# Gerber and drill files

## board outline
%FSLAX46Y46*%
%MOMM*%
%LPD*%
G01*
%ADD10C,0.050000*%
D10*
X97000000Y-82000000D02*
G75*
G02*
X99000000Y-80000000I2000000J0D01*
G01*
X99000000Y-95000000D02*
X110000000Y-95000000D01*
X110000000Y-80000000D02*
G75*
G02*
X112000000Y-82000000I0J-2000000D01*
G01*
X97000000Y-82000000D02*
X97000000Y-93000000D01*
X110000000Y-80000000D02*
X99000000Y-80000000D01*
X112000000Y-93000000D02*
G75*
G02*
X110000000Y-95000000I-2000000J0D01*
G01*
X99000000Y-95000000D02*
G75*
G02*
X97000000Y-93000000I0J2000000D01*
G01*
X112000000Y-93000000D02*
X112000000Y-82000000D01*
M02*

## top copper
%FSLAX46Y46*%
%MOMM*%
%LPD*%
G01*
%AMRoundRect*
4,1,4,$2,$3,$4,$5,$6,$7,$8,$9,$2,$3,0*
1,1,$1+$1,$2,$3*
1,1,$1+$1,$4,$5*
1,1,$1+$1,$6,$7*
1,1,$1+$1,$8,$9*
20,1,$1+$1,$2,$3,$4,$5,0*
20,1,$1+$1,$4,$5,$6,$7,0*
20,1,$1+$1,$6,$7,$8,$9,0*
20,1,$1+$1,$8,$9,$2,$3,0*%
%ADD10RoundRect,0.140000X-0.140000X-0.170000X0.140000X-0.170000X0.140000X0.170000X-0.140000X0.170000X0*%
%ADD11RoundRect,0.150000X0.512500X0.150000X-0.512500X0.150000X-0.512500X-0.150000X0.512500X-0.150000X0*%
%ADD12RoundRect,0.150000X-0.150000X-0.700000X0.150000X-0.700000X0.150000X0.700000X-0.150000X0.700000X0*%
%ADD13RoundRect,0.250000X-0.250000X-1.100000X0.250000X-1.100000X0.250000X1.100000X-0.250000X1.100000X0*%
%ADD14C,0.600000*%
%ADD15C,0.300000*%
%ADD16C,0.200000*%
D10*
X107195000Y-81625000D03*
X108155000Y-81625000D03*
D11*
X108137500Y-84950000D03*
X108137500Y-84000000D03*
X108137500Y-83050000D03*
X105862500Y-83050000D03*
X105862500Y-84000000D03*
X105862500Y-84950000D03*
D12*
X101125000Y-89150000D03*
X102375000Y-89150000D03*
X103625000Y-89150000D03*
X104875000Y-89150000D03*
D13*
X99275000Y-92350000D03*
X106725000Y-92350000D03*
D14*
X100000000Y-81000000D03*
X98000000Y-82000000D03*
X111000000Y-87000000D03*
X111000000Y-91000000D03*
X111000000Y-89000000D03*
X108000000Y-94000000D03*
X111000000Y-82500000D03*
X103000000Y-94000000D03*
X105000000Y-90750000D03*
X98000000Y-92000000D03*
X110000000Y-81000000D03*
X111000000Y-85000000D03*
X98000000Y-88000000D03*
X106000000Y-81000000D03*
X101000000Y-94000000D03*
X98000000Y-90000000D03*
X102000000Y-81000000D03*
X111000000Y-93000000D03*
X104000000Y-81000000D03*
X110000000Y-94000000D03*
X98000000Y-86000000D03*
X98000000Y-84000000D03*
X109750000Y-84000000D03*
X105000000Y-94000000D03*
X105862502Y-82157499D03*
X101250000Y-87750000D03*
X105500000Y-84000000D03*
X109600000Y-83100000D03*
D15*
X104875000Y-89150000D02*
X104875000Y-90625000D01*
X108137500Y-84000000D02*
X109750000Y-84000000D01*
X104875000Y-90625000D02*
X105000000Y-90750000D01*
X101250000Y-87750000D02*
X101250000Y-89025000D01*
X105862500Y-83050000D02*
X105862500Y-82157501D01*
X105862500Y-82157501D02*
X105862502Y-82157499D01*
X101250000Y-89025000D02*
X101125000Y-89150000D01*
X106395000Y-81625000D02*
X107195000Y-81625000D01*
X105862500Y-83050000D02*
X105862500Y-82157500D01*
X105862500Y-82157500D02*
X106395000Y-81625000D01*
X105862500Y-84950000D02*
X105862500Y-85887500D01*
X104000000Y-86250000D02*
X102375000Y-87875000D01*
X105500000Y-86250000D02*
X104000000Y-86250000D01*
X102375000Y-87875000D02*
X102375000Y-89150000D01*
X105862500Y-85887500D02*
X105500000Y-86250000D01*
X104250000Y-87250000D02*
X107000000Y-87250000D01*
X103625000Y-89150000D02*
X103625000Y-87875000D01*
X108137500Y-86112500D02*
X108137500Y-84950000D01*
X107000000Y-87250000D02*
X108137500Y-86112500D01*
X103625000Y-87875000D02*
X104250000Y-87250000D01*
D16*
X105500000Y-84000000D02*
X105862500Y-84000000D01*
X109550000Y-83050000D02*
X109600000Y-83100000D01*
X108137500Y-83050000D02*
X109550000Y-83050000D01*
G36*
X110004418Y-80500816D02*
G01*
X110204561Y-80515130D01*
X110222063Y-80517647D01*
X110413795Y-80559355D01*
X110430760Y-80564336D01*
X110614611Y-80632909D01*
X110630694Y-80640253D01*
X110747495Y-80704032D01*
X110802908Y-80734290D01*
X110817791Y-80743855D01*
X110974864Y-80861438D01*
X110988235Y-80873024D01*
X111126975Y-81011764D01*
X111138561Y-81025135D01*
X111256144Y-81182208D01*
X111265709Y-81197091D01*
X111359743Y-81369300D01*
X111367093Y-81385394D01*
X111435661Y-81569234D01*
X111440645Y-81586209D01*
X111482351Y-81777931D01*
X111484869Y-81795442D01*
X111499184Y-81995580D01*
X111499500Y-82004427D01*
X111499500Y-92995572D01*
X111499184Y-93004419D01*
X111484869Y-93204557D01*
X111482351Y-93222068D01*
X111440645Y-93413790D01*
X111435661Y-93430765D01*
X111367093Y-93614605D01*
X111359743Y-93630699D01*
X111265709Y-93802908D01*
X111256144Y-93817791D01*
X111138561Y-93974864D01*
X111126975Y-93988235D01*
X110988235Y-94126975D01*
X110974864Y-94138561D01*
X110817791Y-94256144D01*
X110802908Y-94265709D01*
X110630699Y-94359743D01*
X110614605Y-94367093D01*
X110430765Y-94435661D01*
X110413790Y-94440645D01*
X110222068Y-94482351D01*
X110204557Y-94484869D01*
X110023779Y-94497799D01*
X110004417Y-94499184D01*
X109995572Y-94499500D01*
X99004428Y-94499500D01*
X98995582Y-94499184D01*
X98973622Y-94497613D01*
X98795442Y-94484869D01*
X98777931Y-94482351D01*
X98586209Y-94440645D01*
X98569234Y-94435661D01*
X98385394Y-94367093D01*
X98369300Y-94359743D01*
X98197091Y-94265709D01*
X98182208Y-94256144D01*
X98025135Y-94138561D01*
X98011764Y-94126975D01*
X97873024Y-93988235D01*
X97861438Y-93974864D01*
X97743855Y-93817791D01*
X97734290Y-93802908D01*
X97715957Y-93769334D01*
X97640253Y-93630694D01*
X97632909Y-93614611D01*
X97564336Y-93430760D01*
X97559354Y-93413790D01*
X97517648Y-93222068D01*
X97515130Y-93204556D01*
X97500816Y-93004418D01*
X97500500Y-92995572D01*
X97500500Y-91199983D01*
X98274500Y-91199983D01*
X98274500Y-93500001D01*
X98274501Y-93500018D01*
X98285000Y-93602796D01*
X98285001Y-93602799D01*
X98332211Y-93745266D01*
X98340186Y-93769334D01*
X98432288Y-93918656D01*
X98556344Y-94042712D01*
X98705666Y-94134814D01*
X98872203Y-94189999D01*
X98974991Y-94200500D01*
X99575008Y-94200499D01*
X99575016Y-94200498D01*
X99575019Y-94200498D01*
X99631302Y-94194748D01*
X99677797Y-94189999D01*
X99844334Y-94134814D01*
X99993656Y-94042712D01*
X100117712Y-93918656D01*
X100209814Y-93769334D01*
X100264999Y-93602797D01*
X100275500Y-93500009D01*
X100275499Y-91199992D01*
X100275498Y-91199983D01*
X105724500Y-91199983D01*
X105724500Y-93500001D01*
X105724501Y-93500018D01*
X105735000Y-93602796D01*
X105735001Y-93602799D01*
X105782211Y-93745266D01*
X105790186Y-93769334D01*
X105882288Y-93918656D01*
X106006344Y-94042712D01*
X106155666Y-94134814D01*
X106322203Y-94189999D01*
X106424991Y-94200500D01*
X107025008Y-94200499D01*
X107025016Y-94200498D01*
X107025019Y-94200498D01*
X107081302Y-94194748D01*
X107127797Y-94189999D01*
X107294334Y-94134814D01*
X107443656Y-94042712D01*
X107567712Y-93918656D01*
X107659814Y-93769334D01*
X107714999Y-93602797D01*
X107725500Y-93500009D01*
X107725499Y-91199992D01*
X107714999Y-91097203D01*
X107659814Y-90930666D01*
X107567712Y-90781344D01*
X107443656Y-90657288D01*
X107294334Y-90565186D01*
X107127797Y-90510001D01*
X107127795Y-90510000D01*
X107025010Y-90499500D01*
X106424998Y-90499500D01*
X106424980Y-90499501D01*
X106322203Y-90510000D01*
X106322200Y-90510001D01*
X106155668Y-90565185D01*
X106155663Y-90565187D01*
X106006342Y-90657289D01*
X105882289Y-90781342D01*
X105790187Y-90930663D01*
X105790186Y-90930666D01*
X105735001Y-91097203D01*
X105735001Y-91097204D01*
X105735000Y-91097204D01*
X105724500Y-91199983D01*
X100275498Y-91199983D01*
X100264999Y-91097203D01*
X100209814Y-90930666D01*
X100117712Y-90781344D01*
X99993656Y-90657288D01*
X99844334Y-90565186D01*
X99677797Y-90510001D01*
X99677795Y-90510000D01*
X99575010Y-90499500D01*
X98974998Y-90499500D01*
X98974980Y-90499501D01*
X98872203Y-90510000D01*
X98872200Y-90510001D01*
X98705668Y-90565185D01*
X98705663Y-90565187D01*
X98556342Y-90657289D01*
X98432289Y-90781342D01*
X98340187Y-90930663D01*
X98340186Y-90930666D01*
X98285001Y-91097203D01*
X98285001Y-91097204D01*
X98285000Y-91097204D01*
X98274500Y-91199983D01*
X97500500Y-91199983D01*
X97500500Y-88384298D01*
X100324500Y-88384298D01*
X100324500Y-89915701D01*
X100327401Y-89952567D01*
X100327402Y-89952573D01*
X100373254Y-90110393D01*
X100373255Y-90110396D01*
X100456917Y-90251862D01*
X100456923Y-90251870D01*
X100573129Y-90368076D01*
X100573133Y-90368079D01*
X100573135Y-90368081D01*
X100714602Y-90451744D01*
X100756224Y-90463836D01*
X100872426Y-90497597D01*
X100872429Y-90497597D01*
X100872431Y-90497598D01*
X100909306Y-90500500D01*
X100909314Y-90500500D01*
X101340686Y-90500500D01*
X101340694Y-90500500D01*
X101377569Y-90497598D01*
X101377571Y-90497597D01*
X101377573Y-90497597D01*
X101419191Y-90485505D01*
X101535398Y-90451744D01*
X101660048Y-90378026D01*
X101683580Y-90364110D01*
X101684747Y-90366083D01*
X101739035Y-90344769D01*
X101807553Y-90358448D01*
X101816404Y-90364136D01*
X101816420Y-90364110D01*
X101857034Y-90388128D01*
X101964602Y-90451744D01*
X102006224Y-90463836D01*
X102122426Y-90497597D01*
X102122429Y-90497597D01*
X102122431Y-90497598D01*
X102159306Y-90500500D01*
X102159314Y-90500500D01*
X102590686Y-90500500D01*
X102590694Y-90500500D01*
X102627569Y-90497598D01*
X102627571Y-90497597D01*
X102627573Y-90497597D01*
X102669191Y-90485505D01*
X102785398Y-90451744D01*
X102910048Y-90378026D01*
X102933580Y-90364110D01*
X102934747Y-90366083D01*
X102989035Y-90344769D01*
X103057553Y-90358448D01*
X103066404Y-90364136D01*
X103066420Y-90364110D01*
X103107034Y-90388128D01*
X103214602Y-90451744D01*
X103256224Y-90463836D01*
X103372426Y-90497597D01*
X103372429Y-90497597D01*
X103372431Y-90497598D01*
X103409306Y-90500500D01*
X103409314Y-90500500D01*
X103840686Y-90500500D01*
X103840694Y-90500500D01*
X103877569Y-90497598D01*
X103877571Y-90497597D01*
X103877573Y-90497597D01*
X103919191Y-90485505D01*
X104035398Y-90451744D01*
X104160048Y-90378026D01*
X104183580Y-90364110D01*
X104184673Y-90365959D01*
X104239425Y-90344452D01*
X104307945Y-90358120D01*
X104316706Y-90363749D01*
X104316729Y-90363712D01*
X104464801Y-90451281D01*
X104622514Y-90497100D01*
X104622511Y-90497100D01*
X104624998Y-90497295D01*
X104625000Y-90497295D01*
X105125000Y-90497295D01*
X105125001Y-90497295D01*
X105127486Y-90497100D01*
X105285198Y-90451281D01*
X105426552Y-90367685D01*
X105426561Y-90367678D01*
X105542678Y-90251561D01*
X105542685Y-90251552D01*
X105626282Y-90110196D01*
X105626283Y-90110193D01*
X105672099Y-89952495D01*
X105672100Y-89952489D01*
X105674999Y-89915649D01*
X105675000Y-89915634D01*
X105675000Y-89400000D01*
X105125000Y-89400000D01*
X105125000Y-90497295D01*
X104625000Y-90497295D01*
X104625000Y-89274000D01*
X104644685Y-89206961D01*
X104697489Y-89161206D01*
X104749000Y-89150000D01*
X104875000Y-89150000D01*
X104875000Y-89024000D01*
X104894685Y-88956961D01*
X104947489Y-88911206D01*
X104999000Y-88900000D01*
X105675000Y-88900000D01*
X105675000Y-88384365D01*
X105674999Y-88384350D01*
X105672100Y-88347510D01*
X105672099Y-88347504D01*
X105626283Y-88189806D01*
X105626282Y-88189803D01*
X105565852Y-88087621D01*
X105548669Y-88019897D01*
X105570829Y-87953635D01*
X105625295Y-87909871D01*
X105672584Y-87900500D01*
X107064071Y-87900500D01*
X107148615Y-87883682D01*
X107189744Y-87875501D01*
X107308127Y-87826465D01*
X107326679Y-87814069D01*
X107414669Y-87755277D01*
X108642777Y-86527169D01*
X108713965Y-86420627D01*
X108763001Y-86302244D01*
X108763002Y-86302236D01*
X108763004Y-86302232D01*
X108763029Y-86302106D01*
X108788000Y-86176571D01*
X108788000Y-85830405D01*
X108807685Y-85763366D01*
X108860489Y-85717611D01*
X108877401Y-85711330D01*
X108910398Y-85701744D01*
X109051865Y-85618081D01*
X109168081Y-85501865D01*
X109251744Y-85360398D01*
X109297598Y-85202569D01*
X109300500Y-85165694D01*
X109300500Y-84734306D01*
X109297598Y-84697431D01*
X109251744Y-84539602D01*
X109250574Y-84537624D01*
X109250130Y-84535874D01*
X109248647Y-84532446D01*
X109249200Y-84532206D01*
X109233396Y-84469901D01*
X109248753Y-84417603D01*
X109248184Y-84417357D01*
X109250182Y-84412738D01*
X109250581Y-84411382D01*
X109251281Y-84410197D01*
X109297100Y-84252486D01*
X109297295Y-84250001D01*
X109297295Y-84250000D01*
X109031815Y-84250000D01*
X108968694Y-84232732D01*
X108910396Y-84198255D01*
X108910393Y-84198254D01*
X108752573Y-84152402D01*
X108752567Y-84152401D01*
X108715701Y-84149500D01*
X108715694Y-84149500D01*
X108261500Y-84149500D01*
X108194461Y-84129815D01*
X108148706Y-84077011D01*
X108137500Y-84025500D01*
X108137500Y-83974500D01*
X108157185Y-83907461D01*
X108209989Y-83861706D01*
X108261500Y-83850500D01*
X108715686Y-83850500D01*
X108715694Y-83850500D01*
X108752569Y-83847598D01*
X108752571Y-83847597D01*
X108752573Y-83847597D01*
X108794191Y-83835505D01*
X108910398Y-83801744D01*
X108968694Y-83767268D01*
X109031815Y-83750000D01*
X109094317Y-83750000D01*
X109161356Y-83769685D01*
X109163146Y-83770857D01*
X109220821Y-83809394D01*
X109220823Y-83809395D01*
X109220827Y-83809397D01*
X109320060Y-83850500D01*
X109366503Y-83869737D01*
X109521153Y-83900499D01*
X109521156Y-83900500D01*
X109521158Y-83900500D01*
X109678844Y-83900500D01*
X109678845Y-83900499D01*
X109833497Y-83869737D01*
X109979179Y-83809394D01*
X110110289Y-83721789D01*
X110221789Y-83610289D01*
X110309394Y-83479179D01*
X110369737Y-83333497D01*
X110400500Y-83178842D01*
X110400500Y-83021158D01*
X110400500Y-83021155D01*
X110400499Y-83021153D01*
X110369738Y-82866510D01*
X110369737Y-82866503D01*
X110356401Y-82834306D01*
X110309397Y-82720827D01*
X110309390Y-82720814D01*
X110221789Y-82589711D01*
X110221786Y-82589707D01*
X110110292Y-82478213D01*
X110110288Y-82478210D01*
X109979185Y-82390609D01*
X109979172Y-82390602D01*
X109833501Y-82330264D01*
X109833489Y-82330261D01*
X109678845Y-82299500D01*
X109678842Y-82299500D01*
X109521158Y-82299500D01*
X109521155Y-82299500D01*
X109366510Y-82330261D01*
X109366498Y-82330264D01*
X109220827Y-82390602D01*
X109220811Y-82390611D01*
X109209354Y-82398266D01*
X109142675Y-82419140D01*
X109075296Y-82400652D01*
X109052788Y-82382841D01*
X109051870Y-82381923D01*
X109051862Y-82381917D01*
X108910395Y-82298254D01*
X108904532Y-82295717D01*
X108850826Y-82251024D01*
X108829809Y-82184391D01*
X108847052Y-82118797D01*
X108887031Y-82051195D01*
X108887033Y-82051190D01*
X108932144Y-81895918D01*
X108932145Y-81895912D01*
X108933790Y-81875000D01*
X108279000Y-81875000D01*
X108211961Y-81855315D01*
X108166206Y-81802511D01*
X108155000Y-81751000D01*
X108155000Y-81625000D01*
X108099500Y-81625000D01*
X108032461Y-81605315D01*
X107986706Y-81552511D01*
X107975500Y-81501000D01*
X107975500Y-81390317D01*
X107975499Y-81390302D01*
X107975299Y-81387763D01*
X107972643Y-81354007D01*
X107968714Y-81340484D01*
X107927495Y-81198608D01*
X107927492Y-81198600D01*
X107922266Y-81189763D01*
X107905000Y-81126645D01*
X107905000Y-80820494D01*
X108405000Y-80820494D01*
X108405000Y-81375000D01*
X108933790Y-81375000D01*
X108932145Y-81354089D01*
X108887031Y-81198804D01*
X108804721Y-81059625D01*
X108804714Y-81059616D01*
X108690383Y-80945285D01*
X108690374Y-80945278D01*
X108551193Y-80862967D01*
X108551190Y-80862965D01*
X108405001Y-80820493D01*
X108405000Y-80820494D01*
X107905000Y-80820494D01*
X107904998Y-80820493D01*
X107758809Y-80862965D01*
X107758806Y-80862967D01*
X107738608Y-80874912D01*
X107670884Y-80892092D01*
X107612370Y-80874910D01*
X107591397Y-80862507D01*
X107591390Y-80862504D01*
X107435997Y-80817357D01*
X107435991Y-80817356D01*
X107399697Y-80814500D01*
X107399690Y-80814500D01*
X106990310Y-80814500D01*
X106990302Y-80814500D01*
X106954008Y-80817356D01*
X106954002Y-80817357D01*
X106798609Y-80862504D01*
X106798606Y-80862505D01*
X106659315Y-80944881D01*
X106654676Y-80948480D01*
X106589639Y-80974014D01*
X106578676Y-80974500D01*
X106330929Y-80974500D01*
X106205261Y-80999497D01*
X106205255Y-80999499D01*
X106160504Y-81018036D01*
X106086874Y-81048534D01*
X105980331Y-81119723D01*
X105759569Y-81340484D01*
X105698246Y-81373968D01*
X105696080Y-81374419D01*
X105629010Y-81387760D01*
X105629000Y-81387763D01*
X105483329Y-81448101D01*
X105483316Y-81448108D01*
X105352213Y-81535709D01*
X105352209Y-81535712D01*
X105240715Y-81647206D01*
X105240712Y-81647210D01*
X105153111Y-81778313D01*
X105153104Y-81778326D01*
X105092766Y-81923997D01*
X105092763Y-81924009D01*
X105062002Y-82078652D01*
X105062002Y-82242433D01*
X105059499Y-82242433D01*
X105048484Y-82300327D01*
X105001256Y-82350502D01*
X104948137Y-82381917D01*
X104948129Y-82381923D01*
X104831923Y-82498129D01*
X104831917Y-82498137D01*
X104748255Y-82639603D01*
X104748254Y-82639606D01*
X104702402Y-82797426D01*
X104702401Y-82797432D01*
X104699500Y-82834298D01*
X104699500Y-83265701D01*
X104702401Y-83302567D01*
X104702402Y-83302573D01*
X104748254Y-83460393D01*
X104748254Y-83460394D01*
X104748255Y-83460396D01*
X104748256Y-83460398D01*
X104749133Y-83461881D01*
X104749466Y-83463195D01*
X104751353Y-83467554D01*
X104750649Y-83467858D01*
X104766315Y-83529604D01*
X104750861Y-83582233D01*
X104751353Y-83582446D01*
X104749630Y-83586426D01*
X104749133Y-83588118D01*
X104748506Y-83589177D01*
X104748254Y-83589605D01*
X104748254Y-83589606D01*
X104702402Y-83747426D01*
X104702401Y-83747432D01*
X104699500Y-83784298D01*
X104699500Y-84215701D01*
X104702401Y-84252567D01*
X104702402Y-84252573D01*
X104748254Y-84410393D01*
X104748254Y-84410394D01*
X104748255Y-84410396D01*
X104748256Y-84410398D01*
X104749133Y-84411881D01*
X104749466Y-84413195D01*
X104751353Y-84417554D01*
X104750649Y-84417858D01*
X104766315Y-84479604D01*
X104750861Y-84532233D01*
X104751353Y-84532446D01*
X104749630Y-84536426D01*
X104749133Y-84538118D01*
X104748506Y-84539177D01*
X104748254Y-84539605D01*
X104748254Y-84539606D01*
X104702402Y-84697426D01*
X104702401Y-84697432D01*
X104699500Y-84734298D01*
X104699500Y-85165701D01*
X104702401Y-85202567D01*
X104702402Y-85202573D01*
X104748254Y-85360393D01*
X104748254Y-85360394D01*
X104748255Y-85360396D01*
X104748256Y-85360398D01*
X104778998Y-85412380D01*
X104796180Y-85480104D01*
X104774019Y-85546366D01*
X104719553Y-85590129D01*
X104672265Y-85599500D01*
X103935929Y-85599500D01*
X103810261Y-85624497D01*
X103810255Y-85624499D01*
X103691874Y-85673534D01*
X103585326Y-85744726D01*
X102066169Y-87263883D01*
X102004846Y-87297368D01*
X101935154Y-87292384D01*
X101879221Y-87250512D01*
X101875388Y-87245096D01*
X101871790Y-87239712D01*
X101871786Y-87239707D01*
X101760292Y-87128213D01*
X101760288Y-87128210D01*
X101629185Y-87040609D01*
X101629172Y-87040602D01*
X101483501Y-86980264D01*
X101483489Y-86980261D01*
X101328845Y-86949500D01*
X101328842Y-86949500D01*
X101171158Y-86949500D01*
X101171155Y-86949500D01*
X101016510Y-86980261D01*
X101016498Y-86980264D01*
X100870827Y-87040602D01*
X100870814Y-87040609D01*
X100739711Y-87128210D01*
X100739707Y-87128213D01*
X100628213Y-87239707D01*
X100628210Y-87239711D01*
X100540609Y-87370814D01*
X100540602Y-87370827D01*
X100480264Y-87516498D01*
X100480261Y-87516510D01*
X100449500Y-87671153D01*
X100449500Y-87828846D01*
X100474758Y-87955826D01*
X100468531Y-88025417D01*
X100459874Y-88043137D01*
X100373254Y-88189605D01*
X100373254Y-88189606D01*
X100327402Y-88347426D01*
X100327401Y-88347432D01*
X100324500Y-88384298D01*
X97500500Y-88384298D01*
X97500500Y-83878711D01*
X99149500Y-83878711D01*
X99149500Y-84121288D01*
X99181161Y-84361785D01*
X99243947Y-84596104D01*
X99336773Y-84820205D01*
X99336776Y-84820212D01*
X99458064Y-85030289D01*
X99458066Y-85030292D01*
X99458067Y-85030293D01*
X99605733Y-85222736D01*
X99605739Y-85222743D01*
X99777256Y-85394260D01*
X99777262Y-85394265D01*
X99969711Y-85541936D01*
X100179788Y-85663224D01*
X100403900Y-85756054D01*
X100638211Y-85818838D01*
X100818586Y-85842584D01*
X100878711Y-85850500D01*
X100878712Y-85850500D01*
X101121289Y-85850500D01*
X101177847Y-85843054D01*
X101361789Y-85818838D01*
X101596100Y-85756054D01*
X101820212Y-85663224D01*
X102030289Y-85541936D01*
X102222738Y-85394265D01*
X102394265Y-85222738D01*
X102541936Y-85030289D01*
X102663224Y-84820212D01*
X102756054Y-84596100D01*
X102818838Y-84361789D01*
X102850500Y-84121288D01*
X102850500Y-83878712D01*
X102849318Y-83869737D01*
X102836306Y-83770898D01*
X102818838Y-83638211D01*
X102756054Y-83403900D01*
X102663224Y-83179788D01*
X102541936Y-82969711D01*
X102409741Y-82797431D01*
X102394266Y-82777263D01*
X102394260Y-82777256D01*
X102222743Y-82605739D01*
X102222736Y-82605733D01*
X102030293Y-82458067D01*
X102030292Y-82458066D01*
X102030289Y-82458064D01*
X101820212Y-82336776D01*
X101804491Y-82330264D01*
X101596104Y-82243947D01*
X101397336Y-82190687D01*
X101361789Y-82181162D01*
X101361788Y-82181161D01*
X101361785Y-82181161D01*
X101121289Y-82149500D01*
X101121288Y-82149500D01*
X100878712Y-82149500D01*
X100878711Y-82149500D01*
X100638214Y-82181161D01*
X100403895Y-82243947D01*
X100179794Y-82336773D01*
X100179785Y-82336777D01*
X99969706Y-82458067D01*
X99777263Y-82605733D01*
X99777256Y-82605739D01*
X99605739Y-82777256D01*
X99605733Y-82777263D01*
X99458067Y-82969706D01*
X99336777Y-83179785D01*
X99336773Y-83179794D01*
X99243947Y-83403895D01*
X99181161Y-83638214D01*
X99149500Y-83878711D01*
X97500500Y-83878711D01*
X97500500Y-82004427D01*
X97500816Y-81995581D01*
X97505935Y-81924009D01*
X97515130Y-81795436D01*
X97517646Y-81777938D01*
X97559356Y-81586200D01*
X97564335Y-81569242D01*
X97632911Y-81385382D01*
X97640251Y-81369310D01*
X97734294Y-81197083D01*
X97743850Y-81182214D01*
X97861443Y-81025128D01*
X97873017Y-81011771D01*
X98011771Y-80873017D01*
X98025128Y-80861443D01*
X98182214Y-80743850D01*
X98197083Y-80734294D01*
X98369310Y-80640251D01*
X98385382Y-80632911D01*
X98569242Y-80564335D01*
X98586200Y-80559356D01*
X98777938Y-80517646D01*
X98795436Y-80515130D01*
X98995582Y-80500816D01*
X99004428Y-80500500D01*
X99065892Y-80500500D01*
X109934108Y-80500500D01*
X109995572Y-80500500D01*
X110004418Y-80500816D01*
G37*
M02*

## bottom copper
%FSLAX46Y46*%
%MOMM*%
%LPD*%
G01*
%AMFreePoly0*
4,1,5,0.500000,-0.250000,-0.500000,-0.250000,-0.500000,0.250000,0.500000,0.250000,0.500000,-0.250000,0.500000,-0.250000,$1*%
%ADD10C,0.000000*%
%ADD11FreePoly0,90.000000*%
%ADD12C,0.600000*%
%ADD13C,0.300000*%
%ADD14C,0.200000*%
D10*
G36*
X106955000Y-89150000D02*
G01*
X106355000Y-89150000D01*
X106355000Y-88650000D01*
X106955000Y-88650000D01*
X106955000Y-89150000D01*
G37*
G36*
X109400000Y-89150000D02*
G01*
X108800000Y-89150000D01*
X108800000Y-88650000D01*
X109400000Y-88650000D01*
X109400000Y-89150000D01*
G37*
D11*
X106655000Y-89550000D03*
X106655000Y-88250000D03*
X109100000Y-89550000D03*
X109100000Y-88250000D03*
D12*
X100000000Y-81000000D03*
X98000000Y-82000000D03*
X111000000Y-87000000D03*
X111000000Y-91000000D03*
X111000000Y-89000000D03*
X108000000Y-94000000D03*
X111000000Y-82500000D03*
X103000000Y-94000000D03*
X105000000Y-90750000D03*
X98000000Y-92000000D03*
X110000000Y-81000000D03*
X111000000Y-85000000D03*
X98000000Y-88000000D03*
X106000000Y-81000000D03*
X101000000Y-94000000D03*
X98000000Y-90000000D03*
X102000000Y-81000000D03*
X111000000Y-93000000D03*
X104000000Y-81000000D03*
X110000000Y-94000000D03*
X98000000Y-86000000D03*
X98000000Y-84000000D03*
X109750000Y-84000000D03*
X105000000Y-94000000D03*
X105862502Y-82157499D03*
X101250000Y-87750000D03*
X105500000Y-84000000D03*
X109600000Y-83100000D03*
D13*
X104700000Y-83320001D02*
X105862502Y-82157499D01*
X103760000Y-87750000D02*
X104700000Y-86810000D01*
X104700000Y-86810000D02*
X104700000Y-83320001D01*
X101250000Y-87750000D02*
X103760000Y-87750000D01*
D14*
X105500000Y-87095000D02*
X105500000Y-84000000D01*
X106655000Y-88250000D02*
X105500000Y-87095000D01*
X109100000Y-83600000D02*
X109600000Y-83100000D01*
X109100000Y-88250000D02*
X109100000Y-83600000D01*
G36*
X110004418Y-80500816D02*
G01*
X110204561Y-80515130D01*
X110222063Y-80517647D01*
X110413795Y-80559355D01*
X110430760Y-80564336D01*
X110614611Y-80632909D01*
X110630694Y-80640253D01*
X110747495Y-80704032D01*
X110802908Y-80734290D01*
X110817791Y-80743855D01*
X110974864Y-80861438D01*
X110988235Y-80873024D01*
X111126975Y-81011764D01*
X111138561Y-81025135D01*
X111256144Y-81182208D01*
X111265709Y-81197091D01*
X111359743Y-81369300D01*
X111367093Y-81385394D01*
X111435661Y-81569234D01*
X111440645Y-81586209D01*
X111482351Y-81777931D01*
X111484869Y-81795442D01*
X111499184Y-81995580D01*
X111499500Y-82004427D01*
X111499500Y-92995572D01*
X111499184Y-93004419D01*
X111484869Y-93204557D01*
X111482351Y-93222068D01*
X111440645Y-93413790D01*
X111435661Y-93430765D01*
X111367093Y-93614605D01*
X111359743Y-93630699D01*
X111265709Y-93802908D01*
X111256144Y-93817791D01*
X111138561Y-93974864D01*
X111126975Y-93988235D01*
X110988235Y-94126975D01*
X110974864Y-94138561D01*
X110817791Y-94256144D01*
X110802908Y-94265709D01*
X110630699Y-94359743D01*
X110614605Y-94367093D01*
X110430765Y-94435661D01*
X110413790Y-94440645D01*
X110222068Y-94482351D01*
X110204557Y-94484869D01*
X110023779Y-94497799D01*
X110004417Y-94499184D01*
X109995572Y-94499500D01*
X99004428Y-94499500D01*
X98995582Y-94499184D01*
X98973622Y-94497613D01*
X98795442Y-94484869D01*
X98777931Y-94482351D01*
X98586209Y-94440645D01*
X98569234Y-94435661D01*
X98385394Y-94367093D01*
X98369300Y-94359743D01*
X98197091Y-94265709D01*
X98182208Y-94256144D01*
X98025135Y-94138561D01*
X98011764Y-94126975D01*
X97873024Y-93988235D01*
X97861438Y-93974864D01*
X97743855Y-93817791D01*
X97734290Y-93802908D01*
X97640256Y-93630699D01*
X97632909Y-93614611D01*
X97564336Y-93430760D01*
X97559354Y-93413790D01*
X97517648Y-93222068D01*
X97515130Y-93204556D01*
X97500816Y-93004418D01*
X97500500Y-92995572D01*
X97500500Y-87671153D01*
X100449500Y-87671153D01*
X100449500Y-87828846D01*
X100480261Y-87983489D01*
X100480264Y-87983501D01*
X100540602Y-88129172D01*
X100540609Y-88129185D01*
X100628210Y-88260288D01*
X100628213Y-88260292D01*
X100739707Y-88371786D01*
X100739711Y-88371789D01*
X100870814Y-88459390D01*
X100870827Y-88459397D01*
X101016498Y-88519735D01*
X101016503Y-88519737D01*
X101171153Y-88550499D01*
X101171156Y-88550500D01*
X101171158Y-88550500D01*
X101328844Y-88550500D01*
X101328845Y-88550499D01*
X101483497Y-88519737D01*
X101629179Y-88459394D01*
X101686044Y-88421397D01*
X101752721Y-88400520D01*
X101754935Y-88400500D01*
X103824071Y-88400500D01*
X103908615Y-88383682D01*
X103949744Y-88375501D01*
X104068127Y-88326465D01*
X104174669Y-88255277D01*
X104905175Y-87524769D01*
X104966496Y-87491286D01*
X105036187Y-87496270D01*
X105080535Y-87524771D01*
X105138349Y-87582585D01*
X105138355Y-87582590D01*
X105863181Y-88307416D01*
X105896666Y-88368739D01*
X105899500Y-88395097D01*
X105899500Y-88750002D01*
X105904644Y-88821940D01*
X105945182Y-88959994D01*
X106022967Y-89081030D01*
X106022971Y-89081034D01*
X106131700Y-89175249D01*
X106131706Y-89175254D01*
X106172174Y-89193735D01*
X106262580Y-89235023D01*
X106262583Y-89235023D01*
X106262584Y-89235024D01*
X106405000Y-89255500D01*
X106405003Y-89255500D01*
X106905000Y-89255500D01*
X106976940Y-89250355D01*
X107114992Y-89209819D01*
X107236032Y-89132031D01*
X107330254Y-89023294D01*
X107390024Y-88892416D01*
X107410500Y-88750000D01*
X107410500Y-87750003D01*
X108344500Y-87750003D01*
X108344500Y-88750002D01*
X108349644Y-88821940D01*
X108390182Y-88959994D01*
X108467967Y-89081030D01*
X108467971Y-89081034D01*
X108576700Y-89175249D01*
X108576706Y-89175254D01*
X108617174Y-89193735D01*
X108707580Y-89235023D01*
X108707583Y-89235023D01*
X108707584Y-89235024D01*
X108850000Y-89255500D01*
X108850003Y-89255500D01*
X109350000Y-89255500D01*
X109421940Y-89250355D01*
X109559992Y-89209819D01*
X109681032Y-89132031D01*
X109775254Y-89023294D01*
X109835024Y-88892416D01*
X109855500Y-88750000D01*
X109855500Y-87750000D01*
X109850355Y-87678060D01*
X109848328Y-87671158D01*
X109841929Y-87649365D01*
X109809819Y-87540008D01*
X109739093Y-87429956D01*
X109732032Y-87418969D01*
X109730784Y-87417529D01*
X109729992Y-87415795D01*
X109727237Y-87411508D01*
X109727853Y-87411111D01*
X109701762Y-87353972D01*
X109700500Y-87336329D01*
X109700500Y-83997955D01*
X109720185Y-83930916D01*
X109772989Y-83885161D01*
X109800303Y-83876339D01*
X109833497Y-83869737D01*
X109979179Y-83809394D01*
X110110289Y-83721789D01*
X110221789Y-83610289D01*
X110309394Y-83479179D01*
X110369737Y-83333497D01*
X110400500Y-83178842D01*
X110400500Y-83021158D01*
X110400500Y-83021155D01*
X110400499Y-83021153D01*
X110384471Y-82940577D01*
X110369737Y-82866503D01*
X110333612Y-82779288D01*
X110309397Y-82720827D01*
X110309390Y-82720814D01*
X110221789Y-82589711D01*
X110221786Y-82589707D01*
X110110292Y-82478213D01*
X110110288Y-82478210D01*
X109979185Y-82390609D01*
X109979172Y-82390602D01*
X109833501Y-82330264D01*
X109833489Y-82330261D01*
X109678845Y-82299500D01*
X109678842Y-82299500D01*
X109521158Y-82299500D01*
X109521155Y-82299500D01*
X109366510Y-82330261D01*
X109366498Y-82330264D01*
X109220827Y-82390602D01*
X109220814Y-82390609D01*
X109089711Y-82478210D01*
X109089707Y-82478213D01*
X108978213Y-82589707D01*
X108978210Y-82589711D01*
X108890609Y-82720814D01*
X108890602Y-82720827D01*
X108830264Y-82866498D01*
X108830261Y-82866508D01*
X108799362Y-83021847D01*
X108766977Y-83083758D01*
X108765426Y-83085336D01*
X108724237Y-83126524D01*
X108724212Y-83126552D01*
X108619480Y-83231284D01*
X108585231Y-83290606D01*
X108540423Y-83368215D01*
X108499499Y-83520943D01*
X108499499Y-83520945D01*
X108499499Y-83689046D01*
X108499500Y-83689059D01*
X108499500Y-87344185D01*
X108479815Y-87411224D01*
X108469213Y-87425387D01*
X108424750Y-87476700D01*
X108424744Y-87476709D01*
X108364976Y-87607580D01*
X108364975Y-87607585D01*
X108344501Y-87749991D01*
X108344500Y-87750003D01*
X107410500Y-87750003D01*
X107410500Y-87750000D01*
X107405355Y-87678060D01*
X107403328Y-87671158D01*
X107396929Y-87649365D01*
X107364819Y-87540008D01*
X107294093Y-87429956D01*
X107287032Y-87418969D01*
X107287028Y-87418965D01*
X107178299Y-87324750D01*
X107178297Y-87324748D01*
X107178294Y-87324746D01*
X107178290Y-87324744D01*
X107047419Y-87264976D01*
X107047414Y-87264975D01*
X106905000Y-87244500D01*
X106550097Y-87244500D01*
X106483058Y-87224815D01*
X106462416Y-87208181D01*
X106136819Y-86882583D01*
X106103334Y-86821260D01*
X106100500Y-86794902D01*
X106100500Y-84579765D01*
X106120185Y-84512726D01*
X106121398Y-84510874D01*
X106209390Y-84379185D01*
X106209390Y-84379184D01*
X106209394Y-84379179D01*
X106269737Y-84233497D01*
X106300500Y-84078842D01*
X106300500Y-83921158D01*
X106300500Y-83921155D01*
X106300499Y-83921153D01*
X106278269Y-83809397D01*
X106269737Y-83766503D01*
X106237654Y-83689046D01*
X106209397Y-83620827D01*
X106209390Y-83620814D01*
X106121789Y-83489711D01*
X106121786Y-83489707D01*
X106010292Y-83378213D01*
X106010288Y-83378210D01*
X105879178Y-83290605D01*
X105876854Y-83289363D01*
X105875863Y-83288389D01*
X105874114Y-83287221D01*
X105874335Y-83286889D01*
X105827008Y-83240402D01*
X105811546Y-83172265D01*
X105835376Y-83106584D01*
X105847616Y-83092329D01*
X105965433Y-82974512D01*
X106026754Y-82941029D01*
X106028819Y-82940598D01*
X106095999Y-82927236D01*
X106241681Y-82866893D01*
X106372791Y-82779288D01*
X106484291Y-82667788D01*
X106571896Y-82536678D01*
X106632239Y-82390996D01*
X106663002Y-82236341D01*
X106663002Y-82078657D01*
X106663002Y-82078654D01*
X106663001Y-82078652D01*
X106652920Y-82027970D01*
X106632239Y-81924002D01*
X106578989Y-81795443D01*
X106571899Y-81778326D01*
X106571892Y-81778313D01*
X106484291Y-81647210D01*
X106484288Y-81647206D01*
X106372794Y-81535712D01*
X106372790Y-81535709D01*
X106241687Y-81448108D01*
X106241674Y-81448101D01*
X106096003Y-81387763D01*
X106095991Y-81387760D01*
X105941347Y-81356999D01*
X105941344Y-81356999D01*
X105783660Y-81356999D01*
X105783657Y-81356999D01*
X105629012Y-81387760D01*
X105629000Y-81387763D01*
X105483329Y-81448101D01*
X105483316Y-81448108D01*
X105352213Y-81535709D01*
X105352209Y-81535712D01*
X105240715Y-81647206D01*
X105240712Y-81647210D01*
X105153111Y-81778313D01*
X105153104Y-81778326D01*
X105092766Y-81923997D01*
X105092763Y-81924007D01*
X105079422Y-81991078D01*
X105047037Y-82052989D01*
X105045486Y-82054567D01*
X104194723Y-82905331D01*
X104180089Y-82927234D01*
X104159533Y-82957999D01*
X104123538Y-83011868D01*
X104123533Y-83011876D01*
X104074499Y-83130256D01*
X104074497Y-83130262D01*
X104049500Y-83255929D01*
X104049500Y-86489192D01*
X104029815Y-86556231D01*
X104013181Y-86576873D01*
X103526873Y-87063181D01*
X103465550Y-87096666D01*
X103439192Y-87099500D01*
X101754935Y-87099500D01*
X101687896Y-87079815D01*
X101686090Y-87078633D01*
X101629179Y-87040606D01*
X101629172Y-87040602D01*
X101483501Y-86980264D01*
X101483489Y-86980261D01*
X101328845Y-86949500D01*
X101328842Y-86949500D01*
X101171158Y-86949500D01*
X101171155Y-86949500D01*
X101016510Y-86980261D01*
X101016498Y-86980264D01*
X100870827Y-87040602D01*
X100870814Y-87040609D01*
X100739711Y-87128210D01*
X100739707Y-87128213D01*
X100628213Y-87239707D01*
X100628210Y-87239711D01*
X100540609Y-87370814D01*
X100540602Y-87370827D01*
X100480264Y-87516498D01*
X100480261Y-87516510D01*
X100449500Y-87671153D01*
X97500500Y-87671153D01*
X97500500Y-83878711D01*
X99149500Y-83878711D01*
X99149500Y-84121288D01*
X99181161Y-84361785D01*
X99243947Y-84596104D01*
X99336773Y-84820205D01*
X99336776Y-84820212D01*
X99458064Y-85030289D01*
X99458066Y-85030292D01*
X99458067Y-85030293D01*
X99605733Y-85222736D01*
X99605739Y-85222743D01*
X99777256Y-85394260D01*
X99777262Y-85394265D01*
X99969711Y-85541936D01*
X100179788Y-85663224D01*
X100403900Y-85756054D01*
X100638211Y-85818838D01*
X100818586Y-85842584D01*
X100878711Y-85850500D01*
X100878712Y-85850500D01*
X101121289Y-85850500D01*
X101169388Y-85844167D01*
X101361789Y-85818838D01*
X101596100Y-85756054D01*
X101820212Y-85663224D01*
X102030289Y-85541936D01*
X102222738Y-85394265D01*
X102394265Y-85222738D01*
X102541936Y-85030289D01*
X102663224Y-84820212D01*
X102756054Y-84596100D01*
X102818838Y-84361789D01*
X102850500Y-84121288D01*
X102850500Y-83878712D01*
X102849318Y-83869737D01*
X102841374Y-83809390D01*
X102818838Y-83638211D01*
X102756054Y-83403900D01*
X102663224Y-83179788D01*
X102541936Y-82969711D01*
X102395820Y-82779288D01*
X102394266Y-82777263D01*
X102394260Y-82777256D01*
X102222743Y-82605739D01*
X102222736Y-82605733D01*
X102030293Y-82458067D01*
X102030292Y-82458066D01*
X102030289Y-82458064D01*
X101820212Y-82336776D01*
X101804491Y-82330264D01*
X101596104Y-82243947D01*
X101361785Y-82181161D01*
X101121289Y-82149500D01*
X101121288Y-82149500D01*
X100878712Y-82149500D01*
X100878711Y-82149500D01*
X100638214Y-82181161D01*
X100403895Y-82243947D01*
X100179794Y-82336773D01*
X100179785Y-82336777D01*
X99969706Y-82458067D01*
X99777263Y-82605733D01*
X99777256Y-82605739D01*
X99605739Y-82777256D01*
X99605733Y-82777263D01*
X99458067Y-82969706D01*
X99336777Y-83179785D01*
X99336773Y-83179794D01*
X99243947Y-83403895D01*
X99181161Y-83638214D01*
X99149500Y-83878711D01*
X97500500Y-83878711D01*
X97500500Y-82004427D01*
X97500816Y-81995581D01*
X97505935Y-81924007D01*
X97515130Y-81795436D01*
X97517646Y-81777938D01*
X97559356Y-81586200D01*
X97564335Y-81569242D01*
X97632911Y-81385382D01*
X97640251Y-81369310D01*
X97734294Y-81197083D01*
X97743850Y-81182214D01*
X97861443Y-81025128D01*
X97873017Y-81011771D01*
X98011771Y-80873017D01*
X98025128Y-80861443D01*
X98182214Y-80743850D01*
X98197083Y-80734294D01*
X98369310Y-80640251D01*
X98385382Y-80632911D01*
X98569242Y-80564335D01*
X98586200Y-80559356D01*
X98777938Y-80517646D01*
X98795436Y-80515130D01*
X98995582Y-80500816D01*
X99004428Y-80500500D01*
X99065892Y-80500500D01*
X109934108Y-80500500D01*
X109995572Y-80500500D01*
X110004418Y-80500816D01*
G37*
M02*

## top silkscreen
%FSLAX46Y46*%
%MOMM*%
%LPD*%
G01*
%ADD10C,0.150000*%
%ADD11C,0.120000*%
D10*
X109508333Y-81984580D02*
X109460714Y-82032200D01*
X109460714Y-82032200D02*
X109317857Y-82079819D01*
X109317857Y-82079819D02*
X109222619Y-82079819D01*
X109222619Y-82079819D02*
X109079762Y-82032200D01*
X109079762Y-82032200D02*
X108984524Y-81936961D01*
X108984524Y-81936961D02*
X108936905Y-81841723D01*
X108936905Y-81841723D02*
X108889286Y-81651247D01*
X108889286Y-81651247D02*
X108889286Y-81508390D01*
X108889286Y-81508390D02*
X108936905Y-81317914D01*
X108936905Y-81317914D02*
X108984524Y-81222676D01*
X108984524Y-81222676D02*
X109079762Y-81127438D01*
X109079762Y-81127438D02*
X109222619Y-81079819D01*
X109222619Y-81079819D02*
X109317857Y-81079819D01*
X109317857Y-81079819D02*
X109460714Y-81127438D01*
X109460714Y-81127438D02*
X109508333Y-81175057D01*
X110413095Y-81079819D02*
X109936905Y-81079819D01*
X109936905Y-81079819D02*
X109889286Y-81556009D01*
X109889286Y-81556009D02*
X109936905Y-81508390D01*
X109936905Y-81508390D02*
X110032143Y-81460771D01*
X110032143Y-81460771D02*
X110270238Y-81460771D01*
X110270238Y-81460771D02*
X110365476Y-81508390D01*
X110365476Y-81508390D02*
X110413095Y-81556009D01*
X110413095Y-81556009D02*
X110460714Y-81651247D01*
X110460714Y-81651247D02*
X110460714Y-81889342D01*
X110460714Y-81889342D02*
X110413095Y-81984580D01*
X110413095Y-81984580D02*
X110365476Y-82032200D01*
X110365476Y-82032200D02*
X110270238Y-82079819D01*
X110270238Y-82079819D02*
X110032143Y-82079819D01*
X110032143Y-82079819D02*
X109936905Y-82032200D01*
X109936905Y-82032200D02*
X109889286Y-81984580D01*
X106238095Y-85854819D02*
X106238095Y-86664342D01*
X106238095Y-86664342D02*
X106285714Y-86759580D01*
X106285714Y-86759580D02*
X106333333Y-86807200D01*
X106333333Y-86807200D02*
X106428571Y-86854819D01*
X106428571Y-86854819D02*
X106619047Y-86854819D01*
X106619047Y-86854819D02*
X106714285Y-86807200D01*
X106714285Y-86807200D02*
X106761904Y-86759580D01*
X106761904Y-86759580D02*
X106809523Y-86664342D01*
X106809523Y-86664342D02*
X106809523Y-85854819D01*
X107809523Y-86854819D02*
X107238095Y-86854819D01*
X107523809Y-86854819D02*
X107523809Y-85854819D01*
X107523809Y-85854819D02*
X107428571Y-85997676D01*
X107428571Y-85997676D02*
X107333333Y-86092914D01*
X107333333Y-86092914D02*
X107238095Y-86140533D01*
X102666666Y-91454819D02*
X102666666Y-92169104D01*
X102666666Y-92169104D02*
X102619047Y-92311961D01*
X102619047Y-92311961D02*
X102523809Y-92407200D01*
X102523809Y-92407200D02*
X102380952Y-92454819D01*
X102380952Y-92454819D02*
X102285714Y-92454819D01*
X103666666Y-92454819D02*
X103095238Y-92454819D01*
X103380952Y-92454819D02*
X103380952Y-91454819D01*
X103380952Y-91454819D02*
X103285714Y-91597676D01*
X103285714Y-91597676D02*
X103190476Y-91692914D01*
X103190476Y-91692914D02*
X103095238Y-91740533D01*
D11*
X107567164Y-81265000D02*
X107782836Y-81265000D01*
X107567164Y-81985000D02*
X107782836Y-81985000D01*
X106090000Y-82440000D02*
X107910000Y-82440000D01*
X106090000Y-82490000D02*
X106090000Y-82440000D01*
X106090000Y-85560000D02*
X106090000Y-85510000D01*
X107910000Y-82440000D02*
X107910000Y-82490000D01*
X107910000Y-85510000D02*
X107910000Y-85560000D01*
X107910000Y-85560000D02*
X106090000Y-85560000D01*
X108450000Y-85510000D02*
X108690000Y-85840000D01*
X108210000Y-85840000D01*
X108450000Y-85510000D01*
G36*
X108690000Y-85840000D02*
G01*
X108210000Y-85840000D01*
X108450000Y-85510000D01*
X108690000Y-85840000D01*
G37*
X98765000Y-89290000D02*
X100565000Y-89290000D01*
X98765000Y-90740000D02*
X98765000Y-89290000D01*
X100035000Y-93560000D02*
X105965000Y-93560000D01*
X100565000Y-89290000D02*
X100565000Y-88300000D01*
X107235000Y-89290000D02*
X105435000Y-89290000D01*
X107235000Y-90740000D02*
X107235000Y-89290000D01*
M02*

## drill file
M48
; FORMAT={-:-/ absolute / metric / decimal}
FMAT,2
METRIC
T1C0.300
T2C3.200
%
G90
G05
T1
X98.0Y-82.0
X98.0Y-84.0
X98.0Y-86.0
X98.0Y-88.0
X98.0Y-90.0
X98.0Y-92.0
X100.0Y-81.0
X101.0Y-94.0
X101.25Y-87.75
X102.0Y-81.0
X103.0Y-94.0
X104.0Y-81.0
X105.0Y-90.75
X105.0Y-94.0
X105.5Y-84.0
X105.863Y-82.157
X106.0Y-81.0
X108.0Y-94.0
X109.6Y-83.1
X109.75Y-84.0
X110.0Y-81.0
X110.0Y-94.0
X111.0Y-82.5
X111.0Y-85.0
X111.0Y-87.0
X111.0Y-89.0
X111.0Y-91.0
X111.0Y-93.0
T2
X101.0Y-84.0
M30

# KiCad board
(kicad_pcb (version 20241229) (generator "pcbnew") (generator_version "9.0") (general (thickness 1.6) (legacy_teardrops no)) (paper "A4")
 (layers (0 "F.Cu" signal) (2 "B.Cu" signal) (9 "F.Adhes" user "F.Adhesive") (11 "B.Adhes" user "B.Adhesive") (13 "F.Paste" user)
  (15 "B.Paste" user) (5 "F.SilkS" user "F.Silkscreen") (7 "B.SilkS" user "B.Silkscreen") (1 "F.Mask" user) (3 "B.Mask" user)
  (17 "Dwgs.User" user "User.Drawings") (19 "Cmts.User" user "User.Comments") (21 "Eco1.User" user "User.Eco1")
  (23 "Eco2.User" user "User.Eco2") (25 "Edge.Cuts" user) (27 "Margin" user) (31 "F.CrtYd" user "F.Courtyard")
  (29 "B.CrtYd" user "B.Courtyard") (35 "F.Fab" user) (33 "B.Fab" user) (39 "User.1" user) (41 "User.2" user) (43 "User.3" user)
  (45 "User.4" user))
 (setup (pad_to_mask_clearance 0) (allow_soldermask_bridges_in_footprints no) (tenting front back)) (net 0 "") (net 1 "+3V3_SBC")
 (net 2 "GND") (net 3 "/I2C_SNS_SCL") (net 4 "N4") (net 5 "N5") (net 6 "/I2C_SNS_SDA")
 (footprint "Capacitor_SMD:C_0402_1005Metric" (layer "F.Cu") (at 107.675 81.625)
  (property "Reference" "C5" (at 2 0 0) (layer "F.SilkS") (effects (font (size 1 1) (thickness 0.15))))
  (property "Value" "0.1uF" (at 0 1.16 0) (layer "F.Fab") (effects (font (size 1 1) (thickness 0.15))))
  (fp_line (start -0.107836 -0.36) (end 0.107836 -0.36) (stroke (width 0.12) (type solid)) (layer "F.SilkS"))
  (fp_line (start -0.107836 0.36) (end 0.107836 0.36) (stroke (width 0.12) (type solid)) (layer "F.SilkS"))
  (pad "1" smd roundrect (at -0.48 0) (size 0.56 0.62) (layers "F.Cu" "F.Mask" "F.Paste") (roundrect_rratio 0.25) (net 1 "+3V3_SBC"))
  (pad "2" smd roundrect (at 0.48 0) (size 0.56 0.62) (layers "F.Cu" "F.Mask" "F.Paste") (roundrect_rratio 0.25) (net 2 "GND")))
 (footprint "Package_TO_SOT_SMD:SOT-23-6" (layer "F.Cu") (at 107 84 180)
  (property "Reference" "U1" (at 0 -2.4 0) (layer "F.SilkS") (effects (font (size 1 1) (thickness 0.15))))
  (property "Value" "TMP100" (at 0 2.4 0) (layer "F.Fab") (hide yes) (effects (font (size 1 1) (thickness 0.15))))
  (fp_line (start 0.91 1.56) (end -0.91 1.56) (stroke (width 0.12) (type solid)) (layer "F.SilkS"))
  (fp_line (start 0.91 1.51) (end 0.91 1.56) (stroke (width 0.12) (type solid)) (layer "F.SilkS"))
  (fp_line (start 0.91 -1.56) (end 0.91 -1.51) (stroke (width 0.12) (type solid)) (layer "F.SilkS"))
  (fp_line (start -0.91 1.56) (end -0.91 1.51) (stroke (width 0.12) (type solid)) (layer "F.SilkS"))
  (fp_line (start -0.91 -1.51) (end -0.91 -1.56) (stroke (width 0.12) (type solid)) (layer "F.SilkS"))
  (fp_line (start -0.91 -1.56) (end 0.91 -1.56) (stroke (width 0.12) (type solid)) (layer "F.SilkS"))
  (fp_poly (pts (xy -1.45 -1.51) (xy -1.69 -1.84) (xy -1.21 -1.84)) (stroke (width 0.12) (type solid)) (fill yes) (layer "F.SilkS"))
  (pad "1" smd roundrect (at -1.1375 -0.95 180) (size 1.325 0.6) (layers "F.Cu" "F.Mask" "F.Paste") (roundrect_rratio 0.25)
   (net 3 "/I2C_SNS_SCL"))
  (pad "2" smd roundrect (at -1.1375 0 180) (size 1.325 0.6) (layers "F.Cu" "F.Mask" "F.Paste") (roundrect_rratio 0.25) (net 2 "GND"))
  (pad "3" smd roundrect (at -1.1375 0.95 180) (size 1.325 0.6) (layers "F.Cu" "F.Mask" "F.Paste") (roundrect_rratio 0.25) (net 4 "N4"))
  (pad "4" smd roundrect (at 1.1375 0.95 180) (size 1.325 0.6) (layers "F.Cu" "F.Mask" "F.Paste") (roundrect_rratio 0.25) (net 1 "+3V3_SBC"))
  (pad "5" smd roundrect (at 1.1375 0 180) (size 1.325 0.6) (layers "F.Cu" "F.Mask" "F.Paste") (roundrect_rratio 0.25) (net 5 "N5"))
  (pad "6" smd roundrect (at 1.1375 -0.95 180) (size 1.325 0.6) (layers "F.Cu" "F.Mask" "F.Paste") (roundrect_rratio 0.25)
   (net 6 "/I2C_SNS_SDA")))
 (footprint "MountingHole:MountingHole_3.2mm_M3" (layer "F.Cu") (at 101 84)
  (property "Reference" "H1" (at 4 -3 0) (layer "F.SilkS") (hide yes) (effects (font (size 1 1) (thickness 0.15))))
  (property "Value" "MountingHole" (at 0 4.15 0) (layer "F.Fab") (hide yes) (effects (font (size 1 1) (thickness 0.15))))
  (pad "" np_thru_hole circle (at 0 0) (size 3.2 3.2) (drill 3.2) (layers "*.Cu" "*.Mask")))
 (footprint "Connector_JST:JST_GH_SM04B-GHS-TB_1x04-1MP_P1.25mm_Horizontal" (layer "F.Cu") (at 103 91)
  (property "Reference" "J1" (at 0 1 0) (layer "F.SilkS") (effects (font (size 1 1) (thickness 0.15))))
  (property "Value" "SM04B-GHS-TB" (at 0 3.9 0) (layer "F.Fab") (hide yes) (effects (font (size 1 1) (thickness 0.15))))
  (fp_line (start -4.235 -1.71) (end -2.435 -1.71) (stroke (width 0.12) (type solid)) (layer "F.SilkS"))
  (fp_line (start -4.235 -0.26) (end -4.235 -1.71) (stroke (width 0.12) (type solid)) (layer "F.SilkS"))
  (fp_line (start -2.965 2.56) (end 2.965 2.56) (stroke (width 0.12) (type solid)) (layer "F.SilkS"))
  (fp_line (start -2.435 -1.71) (end -2.435 -2.7) (stroke (width 0.12) (type solid)) (layer "F.SilkS"))
  (fp_line (start 4.235 -1.71) (end 2.435 -1.71) (stroke (width 0.12) (type solid)) (layer "F.SilkS"))
  (fp_line (start 4.235 -0.26) (end 4.235 -1.71) (stroke (width 0.12) (type solid)) (layer "F.SilkS"))
  (pad "1" smd roundrect (at -1.875 -1.85) (size 0.6 1.7) (layers "F.Cu" "F.Mask" "F.Paste") (roundrect_rratio 0.25) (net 1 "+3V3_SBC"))
  (pad "2" smd roundrect (at -0.625 -1.85) (size 0.6 1.7) (layers "F.Cu" "F.Mask" "F.Paste") (roundrect_rratio 0.25) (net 6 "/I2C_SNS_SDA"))
  (pad "3" smd roundrect (at 0.625 -1.85) (size 0.6 1.7) (layers "F.Cu" "F.Mask" "F.Paste") (roundrect_rratio 0.25) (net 3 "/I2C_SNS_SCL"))
  (pad "4" smd roundrect (at 1.875 -1.85) (size 0.6 1.7) (layers "F.Cu" "F.Mask" "F.Paste") (roundrect_rratio 0.25) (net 2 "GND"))
  (pad "MP" smd roundrect (at -3.725 1.35) (size 1 2.7) (layers "F.Cu" "F.Mask" "F.Paste") (roundrect_rratio 0.25))
  (pad "MP" smd roundrect (at 3.725 1.35) (size 1 2.7) (layers "F.Cu" "F.Mask" "F.Paste") (roundrect_rratio 0.25)))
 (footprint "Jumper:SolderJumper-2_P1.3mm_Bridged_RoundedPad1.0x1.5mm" (layer "B.Cu") (at 106.655 88.9 90)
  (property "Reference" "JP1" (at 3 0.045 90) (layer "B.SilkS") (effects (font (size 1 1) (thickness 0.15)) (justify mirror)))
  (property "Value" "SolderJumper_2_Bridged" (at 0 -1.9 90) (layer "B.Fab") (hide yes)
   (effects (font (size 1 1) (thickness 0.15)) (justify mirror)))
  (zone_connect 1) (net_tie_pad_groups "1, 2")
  (fp_poly (pts (xy 0.25 0.3) (xy -0.25 0.3) (xy -0.25 -0.3) (xy 0.25 -0.3)) (stroke (width 0) (type solid)) (fill yes) (layer "B.Cu"))
  (pad "1" smd custom (at -0.65 0 90) (size 1 0.5) (layers "B.Cu" "B.Mask") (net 2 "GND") (zone_connect 2) (thermal_bridge_angle 45)
   (options (clearance outline) (anchor rect)) (primitives))
  (pad "2" smd custom (at 0.65 0 90) (size 1 0.5) (layers "B.Cu" "B.Mask") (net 5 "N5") (zone_connect 2) (thermal_bridge_angle 45)
   (options (clearance outline) (anchor rect)) (primitives)))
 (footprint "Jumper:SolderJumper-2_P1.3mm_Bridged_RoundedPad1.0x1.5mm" (layer "B.Cu") (at 109.1 88.9 90)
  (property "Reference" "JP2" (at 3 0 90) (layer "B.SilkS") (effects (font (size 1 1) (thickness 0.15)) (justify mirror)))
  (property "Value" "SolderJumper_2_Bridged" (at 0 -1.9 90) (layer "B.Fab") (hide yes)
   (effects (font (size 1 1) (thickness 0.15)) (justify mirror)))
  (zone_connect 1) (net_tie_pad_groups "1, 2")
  (fp_poly (pts (xy 0.25 0.3) (xy -0.25 0.3) (xy -0.25 -0.3) (xy 0.25 -0.3)) (stroke (width 0) (type solid)) (fill yes) (layer "B.Cu"))
  (pad "1" smd custom (at -0.65 0 90) (size 1 0.5) (layers "B.Cu" "B.Mask") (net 2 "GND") (zone_connect 2) (thermal_bridge_angle 45)
   (options (clearance outline) (anchor rect)) (primitives))
  (pad "2" smd custom (at 0.65 0 90) (size 1 0.5) (layers "B.Cu" "B.Mask") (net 4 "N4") (zone_connect 2) (thermal_bridge_angle 45)
   (options (clearance outline) (anchor rect)) (primitives)))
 (gr_arc (start 97 82) (mid 97.585786 80.585786) (end 99 80) (stroke (width 0.05) (type default)) (layer "Edge.Cuts"))
 (gr_line (start 99 95) (end 110 95) (stroke (width 0.05) (type default)) (layer "Edge.Cuts"))
 (gr_arc (start 110 80) (mid 111.414214 80.585786) (end 112 82) (stroke (width 0.05) (type default)) (layer "Edge.Cuts"))
 (gr_line (start 97 82) (end 97 93) (stroke (width 0.05) (type default)) (layer "Edge.Cuts"))
 (gr_line (start 110 80) (end 99 80) (stroke (width 0.05) (type default)) (layer "Edge.Cuts"))
 (gr_arc (start 112 93) (mid 111.414214 94.414214) (end 110 95) (stroke (width 0.05) (type default)) (layer "Edge.Cuts"))
 (gr_arc (start 99 95) (mid 97.585786 94.414214) (end 97 93) (stroke (width 0.05) (type default)) (layer "Edge.Cuts"))
 (gr_line (start 112 93) (end 112 82) (stroke (width 0.05) (type default)) (layer "Edge.Cuts"))
 (segment (start 104.875 89.15) (end 104.875 90.625) (width 0.3) (layer "F.Cu") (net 2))
 (segment (start 108.1375 84) (end 109.75 84) (width 0.3) (layer "F.Cu") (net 2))
 (segment (start 104.875 90.625) (end 105 90.75) (width 0.3) (layer "F.Cu") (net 2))
 (via (at 100 81) (size 0.6) (drill 0.3) (layers "F.Cu" "B.Cu") (free yes) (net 2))
 (via (at 98 82) (size 0.6) (drill 0.3) (layers "F.Cu" "B.Cu") (free yes) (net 2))
 (via (at 111 87) (size 0.6) (drill 0.3) (layers "F.Cu" "B.Cu") (free yes) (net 2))
 (via (at 111 91) (size 0.6) (drill 0.3) (layers "F.Cu" "B.Cu") (free yes) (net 2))
 (via (at 111 89) (size 0.6) (drill 0.3) (layers "F.Cu" "B.Cu") (free yes) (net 2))
 (via (at 108 94) (size 0.6) (drill 0.3) (layers "F.Cu" "B.Cu") (free yes) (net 2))
 (via (at 111 82.5) (size 0.6) (drill 0.3) (layers "F.Cu" "B.Cu") (free yes) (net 2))
 (via (at 103 94) (size 0.6) (drill 0.3) (layers "F.Cu" "B.Cu") (free yes) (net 2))
 (via (at 105 90.75) (size 0.6) (drill 0.3) (layers "F.Cu" "B.Cu") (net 2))
 (via (at 98 92) (size 0.6) (drill 0.3) (layers "F.Cu" "B.Cu") (free yes) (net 2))
 (via (at 110 81) (size 0.6) (drill 0.3) (layers "F.Cu" "B.Cu") (free yes) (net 2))
 (via (at 111 85) (size 0.6) (drill 0.3) (layers "F.Cu" "B.Cu") (free yes) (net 2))
 (via (at 98 88) (size 0.6) (drill 0.3) (layers "F.Cu" "B.Cu") (free yes) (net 2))
 (via (at 106 81) (size 0.6) (drill 0.3) (layers "F.Cu" "B.Cu") (free yes) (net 2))
 (via (at 101 94) (size 0.6) (drill 0.3) (layers "F.Cu" "B.Cu") (free yes) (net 2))
 (via (at 98 90) (size 0.6) (drill 0.3) (layers "F.Cu" "B.Cu") (free yes) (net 2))
 (via (at 102 81) (size 0.6) (drill 0.3) (layers "F.Cu" "B.Cu") (free yes) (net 2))
 (via (at 111 93) (size 0.6) (drill 0.3) (layers "F.Cu" "B.Cu") (free yes) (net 2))
 (via (at 104 81) (size 0.6) (drill 0.3) (layers "F.Cu" "B.Cu") (free yes) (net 2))
 (via (at 110 94) (size 0.6) (drill 0.3) (layers "F.Cu" "B.Cu") (free yes) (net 2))
 (via (at 98 86) (size 0.6) (drill 0.3) (layers "F.Cu" "B.Cu") (free yes) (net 2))
 (via (at 98 84) (size 0.6) (drill 0.3) (layers "F.Cu" "B.Cu") (free yes) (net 2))
 (via (at 109.75 84) (size 0.6) (drill 0.3) (layers "F.Cu" "B.Cu") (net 2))
 (via (at 105 94) (size 0.6) (drill 0.3) (layers "F.Cu" "B.Cu") (free yes) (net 2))
 (segment (start 101.25 87.75) (end 101.25 89.025) (width 0.3) (layer "F.Cu") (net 1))
 (segment (start 105.8625 83.05) (end 105.8625 82.157501) (width 0.3) (layer "F.Cu") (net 1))
 (segment (start 105.8625 82.157501) (end 105.862502 82.157499) (width 0.3) (layer "F.Cu") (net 1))
 (segment (start 101.25 89.025) (end 101.125 89.15) (width 0.3) (layer "F.Cu") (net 1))
 (segment (start 106.395 81.625) (end 107.195 81.625) (width 0.3) (layer "F.Cu") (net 1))
 (segment (start 105.8625 83.05) (end 105.8625 82.1575) (width 0.3) (layer "F.Cu") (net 1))
 (segment (start 105.8625 82.1575) (end 106.395 81.625) (width 0.3) (layer "F.Cu") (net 1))
 (via (at 105.862502 82.157499) (size 0.6) (drill 0.3) (layers "F.Cu" "B.Cu") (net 1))
 (via (at 101.25 87.75) (size 0.6) (drill 0.3) (layers "F.Cu" "B.Cu") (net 1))
 (segment (start 104.7 83.320001) (end 105.862502 82.157499) (width 0.3) (layer "B.Cu") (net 1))
 (segment (start 103.76 87.75) (end 104.7 86.81) (width 0.3) (layer "B.Cu") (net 1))
 (segment (start 104.7 86.81) (end 104.7 83.320001) (width 0.3) (layer "B.Cu") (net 1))
 (segment (start 101.25 87.75) (end 103.76 87.75) (width 0.3) (layer "B.Cu") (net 1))
 (segment (start 105.8625 84.95) (end 105.8625 85.8875) (width 0.3) (layer "F.Cu") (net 6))
 (segment (start 104 86.25) (end 102.375 87.875) (width 0.3) (layer "F.Cu") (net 6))
 (segment (start 105.5 86.25) (end 104 86.25) (width 0.3) (layer "F.Cu") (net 6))
 (segment (start 102.375 87.875) (end 102.375 89.15) (width 0.3) (layer "F.Cu") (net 6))
 (segment (start 105.8625 85.8875) (end 105.5 86.25) (width 0.3) (layer "F.Cu") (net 6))
 (segment (start 104.25 87.25) (end 107 87.25) (width 0.3) (layer "F.Cu") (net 3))
 (segment (start 103.625 89.15) (end 103.625 87.875) (width 0.3) (layer "F.Cu") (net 3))
 (segment (start 108.1375 86.1125) (end 108.1375 84.95) (width 0.3) (layer "F.Cu") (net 3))
 (segment (start 107 87.25) (end 108.1375 86.1125) (width 0.3) (layer "F.Cu") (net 3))
 (segment (start 103.625 87.875) (end 104.25 87.25) (width 0.3) (layer "F.Cu") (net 3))
 (segment (start 105.5 84) (end 105.8625 84) (width 0.2) (layer "F.Cu") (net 5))
 (via (at 105.5 84) (size 0.6) (drill 0.3) (layers "F.Cu" "B.Cu") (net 5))
 (segment (start 105.5 87.095) (end 105.5 84) (width 0.2) (layer "B.Cu") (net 5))
 (segment (start 106.655 88.25) (end 105.5 87.095) (width 0.2) (layer "B.Cu") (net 5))
 (segment (start 109.55 83.05) (end 109.6 83.1) (width 0.2) (layer "F.Cu") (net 4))
 (segment (start 108.1375 83.05) (end 109.55 83.05) (width 0.2) (layer "F.Cu") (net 4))
 (via (at 109.6 83.1) (size 0.6) (drill 0.3) (layers "F.Cu" "B.Cu") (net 4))
 (segment (start 109.1 83.6) (end 109.6 83.1) (width 0.2) (layer "B.Cu") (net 4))
 (segment (start 109.1 88.25) (end 109.1 83.6) (width 0.2) (layer "B.Cu") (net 4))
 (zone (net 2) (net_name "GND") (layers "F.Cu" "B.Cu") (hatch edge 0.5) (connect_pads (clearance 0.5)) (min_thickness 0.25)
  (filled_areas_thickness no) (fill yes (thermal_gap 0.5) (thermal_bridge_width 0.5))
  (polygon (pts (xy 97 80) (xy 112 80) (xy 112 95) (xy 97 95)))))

